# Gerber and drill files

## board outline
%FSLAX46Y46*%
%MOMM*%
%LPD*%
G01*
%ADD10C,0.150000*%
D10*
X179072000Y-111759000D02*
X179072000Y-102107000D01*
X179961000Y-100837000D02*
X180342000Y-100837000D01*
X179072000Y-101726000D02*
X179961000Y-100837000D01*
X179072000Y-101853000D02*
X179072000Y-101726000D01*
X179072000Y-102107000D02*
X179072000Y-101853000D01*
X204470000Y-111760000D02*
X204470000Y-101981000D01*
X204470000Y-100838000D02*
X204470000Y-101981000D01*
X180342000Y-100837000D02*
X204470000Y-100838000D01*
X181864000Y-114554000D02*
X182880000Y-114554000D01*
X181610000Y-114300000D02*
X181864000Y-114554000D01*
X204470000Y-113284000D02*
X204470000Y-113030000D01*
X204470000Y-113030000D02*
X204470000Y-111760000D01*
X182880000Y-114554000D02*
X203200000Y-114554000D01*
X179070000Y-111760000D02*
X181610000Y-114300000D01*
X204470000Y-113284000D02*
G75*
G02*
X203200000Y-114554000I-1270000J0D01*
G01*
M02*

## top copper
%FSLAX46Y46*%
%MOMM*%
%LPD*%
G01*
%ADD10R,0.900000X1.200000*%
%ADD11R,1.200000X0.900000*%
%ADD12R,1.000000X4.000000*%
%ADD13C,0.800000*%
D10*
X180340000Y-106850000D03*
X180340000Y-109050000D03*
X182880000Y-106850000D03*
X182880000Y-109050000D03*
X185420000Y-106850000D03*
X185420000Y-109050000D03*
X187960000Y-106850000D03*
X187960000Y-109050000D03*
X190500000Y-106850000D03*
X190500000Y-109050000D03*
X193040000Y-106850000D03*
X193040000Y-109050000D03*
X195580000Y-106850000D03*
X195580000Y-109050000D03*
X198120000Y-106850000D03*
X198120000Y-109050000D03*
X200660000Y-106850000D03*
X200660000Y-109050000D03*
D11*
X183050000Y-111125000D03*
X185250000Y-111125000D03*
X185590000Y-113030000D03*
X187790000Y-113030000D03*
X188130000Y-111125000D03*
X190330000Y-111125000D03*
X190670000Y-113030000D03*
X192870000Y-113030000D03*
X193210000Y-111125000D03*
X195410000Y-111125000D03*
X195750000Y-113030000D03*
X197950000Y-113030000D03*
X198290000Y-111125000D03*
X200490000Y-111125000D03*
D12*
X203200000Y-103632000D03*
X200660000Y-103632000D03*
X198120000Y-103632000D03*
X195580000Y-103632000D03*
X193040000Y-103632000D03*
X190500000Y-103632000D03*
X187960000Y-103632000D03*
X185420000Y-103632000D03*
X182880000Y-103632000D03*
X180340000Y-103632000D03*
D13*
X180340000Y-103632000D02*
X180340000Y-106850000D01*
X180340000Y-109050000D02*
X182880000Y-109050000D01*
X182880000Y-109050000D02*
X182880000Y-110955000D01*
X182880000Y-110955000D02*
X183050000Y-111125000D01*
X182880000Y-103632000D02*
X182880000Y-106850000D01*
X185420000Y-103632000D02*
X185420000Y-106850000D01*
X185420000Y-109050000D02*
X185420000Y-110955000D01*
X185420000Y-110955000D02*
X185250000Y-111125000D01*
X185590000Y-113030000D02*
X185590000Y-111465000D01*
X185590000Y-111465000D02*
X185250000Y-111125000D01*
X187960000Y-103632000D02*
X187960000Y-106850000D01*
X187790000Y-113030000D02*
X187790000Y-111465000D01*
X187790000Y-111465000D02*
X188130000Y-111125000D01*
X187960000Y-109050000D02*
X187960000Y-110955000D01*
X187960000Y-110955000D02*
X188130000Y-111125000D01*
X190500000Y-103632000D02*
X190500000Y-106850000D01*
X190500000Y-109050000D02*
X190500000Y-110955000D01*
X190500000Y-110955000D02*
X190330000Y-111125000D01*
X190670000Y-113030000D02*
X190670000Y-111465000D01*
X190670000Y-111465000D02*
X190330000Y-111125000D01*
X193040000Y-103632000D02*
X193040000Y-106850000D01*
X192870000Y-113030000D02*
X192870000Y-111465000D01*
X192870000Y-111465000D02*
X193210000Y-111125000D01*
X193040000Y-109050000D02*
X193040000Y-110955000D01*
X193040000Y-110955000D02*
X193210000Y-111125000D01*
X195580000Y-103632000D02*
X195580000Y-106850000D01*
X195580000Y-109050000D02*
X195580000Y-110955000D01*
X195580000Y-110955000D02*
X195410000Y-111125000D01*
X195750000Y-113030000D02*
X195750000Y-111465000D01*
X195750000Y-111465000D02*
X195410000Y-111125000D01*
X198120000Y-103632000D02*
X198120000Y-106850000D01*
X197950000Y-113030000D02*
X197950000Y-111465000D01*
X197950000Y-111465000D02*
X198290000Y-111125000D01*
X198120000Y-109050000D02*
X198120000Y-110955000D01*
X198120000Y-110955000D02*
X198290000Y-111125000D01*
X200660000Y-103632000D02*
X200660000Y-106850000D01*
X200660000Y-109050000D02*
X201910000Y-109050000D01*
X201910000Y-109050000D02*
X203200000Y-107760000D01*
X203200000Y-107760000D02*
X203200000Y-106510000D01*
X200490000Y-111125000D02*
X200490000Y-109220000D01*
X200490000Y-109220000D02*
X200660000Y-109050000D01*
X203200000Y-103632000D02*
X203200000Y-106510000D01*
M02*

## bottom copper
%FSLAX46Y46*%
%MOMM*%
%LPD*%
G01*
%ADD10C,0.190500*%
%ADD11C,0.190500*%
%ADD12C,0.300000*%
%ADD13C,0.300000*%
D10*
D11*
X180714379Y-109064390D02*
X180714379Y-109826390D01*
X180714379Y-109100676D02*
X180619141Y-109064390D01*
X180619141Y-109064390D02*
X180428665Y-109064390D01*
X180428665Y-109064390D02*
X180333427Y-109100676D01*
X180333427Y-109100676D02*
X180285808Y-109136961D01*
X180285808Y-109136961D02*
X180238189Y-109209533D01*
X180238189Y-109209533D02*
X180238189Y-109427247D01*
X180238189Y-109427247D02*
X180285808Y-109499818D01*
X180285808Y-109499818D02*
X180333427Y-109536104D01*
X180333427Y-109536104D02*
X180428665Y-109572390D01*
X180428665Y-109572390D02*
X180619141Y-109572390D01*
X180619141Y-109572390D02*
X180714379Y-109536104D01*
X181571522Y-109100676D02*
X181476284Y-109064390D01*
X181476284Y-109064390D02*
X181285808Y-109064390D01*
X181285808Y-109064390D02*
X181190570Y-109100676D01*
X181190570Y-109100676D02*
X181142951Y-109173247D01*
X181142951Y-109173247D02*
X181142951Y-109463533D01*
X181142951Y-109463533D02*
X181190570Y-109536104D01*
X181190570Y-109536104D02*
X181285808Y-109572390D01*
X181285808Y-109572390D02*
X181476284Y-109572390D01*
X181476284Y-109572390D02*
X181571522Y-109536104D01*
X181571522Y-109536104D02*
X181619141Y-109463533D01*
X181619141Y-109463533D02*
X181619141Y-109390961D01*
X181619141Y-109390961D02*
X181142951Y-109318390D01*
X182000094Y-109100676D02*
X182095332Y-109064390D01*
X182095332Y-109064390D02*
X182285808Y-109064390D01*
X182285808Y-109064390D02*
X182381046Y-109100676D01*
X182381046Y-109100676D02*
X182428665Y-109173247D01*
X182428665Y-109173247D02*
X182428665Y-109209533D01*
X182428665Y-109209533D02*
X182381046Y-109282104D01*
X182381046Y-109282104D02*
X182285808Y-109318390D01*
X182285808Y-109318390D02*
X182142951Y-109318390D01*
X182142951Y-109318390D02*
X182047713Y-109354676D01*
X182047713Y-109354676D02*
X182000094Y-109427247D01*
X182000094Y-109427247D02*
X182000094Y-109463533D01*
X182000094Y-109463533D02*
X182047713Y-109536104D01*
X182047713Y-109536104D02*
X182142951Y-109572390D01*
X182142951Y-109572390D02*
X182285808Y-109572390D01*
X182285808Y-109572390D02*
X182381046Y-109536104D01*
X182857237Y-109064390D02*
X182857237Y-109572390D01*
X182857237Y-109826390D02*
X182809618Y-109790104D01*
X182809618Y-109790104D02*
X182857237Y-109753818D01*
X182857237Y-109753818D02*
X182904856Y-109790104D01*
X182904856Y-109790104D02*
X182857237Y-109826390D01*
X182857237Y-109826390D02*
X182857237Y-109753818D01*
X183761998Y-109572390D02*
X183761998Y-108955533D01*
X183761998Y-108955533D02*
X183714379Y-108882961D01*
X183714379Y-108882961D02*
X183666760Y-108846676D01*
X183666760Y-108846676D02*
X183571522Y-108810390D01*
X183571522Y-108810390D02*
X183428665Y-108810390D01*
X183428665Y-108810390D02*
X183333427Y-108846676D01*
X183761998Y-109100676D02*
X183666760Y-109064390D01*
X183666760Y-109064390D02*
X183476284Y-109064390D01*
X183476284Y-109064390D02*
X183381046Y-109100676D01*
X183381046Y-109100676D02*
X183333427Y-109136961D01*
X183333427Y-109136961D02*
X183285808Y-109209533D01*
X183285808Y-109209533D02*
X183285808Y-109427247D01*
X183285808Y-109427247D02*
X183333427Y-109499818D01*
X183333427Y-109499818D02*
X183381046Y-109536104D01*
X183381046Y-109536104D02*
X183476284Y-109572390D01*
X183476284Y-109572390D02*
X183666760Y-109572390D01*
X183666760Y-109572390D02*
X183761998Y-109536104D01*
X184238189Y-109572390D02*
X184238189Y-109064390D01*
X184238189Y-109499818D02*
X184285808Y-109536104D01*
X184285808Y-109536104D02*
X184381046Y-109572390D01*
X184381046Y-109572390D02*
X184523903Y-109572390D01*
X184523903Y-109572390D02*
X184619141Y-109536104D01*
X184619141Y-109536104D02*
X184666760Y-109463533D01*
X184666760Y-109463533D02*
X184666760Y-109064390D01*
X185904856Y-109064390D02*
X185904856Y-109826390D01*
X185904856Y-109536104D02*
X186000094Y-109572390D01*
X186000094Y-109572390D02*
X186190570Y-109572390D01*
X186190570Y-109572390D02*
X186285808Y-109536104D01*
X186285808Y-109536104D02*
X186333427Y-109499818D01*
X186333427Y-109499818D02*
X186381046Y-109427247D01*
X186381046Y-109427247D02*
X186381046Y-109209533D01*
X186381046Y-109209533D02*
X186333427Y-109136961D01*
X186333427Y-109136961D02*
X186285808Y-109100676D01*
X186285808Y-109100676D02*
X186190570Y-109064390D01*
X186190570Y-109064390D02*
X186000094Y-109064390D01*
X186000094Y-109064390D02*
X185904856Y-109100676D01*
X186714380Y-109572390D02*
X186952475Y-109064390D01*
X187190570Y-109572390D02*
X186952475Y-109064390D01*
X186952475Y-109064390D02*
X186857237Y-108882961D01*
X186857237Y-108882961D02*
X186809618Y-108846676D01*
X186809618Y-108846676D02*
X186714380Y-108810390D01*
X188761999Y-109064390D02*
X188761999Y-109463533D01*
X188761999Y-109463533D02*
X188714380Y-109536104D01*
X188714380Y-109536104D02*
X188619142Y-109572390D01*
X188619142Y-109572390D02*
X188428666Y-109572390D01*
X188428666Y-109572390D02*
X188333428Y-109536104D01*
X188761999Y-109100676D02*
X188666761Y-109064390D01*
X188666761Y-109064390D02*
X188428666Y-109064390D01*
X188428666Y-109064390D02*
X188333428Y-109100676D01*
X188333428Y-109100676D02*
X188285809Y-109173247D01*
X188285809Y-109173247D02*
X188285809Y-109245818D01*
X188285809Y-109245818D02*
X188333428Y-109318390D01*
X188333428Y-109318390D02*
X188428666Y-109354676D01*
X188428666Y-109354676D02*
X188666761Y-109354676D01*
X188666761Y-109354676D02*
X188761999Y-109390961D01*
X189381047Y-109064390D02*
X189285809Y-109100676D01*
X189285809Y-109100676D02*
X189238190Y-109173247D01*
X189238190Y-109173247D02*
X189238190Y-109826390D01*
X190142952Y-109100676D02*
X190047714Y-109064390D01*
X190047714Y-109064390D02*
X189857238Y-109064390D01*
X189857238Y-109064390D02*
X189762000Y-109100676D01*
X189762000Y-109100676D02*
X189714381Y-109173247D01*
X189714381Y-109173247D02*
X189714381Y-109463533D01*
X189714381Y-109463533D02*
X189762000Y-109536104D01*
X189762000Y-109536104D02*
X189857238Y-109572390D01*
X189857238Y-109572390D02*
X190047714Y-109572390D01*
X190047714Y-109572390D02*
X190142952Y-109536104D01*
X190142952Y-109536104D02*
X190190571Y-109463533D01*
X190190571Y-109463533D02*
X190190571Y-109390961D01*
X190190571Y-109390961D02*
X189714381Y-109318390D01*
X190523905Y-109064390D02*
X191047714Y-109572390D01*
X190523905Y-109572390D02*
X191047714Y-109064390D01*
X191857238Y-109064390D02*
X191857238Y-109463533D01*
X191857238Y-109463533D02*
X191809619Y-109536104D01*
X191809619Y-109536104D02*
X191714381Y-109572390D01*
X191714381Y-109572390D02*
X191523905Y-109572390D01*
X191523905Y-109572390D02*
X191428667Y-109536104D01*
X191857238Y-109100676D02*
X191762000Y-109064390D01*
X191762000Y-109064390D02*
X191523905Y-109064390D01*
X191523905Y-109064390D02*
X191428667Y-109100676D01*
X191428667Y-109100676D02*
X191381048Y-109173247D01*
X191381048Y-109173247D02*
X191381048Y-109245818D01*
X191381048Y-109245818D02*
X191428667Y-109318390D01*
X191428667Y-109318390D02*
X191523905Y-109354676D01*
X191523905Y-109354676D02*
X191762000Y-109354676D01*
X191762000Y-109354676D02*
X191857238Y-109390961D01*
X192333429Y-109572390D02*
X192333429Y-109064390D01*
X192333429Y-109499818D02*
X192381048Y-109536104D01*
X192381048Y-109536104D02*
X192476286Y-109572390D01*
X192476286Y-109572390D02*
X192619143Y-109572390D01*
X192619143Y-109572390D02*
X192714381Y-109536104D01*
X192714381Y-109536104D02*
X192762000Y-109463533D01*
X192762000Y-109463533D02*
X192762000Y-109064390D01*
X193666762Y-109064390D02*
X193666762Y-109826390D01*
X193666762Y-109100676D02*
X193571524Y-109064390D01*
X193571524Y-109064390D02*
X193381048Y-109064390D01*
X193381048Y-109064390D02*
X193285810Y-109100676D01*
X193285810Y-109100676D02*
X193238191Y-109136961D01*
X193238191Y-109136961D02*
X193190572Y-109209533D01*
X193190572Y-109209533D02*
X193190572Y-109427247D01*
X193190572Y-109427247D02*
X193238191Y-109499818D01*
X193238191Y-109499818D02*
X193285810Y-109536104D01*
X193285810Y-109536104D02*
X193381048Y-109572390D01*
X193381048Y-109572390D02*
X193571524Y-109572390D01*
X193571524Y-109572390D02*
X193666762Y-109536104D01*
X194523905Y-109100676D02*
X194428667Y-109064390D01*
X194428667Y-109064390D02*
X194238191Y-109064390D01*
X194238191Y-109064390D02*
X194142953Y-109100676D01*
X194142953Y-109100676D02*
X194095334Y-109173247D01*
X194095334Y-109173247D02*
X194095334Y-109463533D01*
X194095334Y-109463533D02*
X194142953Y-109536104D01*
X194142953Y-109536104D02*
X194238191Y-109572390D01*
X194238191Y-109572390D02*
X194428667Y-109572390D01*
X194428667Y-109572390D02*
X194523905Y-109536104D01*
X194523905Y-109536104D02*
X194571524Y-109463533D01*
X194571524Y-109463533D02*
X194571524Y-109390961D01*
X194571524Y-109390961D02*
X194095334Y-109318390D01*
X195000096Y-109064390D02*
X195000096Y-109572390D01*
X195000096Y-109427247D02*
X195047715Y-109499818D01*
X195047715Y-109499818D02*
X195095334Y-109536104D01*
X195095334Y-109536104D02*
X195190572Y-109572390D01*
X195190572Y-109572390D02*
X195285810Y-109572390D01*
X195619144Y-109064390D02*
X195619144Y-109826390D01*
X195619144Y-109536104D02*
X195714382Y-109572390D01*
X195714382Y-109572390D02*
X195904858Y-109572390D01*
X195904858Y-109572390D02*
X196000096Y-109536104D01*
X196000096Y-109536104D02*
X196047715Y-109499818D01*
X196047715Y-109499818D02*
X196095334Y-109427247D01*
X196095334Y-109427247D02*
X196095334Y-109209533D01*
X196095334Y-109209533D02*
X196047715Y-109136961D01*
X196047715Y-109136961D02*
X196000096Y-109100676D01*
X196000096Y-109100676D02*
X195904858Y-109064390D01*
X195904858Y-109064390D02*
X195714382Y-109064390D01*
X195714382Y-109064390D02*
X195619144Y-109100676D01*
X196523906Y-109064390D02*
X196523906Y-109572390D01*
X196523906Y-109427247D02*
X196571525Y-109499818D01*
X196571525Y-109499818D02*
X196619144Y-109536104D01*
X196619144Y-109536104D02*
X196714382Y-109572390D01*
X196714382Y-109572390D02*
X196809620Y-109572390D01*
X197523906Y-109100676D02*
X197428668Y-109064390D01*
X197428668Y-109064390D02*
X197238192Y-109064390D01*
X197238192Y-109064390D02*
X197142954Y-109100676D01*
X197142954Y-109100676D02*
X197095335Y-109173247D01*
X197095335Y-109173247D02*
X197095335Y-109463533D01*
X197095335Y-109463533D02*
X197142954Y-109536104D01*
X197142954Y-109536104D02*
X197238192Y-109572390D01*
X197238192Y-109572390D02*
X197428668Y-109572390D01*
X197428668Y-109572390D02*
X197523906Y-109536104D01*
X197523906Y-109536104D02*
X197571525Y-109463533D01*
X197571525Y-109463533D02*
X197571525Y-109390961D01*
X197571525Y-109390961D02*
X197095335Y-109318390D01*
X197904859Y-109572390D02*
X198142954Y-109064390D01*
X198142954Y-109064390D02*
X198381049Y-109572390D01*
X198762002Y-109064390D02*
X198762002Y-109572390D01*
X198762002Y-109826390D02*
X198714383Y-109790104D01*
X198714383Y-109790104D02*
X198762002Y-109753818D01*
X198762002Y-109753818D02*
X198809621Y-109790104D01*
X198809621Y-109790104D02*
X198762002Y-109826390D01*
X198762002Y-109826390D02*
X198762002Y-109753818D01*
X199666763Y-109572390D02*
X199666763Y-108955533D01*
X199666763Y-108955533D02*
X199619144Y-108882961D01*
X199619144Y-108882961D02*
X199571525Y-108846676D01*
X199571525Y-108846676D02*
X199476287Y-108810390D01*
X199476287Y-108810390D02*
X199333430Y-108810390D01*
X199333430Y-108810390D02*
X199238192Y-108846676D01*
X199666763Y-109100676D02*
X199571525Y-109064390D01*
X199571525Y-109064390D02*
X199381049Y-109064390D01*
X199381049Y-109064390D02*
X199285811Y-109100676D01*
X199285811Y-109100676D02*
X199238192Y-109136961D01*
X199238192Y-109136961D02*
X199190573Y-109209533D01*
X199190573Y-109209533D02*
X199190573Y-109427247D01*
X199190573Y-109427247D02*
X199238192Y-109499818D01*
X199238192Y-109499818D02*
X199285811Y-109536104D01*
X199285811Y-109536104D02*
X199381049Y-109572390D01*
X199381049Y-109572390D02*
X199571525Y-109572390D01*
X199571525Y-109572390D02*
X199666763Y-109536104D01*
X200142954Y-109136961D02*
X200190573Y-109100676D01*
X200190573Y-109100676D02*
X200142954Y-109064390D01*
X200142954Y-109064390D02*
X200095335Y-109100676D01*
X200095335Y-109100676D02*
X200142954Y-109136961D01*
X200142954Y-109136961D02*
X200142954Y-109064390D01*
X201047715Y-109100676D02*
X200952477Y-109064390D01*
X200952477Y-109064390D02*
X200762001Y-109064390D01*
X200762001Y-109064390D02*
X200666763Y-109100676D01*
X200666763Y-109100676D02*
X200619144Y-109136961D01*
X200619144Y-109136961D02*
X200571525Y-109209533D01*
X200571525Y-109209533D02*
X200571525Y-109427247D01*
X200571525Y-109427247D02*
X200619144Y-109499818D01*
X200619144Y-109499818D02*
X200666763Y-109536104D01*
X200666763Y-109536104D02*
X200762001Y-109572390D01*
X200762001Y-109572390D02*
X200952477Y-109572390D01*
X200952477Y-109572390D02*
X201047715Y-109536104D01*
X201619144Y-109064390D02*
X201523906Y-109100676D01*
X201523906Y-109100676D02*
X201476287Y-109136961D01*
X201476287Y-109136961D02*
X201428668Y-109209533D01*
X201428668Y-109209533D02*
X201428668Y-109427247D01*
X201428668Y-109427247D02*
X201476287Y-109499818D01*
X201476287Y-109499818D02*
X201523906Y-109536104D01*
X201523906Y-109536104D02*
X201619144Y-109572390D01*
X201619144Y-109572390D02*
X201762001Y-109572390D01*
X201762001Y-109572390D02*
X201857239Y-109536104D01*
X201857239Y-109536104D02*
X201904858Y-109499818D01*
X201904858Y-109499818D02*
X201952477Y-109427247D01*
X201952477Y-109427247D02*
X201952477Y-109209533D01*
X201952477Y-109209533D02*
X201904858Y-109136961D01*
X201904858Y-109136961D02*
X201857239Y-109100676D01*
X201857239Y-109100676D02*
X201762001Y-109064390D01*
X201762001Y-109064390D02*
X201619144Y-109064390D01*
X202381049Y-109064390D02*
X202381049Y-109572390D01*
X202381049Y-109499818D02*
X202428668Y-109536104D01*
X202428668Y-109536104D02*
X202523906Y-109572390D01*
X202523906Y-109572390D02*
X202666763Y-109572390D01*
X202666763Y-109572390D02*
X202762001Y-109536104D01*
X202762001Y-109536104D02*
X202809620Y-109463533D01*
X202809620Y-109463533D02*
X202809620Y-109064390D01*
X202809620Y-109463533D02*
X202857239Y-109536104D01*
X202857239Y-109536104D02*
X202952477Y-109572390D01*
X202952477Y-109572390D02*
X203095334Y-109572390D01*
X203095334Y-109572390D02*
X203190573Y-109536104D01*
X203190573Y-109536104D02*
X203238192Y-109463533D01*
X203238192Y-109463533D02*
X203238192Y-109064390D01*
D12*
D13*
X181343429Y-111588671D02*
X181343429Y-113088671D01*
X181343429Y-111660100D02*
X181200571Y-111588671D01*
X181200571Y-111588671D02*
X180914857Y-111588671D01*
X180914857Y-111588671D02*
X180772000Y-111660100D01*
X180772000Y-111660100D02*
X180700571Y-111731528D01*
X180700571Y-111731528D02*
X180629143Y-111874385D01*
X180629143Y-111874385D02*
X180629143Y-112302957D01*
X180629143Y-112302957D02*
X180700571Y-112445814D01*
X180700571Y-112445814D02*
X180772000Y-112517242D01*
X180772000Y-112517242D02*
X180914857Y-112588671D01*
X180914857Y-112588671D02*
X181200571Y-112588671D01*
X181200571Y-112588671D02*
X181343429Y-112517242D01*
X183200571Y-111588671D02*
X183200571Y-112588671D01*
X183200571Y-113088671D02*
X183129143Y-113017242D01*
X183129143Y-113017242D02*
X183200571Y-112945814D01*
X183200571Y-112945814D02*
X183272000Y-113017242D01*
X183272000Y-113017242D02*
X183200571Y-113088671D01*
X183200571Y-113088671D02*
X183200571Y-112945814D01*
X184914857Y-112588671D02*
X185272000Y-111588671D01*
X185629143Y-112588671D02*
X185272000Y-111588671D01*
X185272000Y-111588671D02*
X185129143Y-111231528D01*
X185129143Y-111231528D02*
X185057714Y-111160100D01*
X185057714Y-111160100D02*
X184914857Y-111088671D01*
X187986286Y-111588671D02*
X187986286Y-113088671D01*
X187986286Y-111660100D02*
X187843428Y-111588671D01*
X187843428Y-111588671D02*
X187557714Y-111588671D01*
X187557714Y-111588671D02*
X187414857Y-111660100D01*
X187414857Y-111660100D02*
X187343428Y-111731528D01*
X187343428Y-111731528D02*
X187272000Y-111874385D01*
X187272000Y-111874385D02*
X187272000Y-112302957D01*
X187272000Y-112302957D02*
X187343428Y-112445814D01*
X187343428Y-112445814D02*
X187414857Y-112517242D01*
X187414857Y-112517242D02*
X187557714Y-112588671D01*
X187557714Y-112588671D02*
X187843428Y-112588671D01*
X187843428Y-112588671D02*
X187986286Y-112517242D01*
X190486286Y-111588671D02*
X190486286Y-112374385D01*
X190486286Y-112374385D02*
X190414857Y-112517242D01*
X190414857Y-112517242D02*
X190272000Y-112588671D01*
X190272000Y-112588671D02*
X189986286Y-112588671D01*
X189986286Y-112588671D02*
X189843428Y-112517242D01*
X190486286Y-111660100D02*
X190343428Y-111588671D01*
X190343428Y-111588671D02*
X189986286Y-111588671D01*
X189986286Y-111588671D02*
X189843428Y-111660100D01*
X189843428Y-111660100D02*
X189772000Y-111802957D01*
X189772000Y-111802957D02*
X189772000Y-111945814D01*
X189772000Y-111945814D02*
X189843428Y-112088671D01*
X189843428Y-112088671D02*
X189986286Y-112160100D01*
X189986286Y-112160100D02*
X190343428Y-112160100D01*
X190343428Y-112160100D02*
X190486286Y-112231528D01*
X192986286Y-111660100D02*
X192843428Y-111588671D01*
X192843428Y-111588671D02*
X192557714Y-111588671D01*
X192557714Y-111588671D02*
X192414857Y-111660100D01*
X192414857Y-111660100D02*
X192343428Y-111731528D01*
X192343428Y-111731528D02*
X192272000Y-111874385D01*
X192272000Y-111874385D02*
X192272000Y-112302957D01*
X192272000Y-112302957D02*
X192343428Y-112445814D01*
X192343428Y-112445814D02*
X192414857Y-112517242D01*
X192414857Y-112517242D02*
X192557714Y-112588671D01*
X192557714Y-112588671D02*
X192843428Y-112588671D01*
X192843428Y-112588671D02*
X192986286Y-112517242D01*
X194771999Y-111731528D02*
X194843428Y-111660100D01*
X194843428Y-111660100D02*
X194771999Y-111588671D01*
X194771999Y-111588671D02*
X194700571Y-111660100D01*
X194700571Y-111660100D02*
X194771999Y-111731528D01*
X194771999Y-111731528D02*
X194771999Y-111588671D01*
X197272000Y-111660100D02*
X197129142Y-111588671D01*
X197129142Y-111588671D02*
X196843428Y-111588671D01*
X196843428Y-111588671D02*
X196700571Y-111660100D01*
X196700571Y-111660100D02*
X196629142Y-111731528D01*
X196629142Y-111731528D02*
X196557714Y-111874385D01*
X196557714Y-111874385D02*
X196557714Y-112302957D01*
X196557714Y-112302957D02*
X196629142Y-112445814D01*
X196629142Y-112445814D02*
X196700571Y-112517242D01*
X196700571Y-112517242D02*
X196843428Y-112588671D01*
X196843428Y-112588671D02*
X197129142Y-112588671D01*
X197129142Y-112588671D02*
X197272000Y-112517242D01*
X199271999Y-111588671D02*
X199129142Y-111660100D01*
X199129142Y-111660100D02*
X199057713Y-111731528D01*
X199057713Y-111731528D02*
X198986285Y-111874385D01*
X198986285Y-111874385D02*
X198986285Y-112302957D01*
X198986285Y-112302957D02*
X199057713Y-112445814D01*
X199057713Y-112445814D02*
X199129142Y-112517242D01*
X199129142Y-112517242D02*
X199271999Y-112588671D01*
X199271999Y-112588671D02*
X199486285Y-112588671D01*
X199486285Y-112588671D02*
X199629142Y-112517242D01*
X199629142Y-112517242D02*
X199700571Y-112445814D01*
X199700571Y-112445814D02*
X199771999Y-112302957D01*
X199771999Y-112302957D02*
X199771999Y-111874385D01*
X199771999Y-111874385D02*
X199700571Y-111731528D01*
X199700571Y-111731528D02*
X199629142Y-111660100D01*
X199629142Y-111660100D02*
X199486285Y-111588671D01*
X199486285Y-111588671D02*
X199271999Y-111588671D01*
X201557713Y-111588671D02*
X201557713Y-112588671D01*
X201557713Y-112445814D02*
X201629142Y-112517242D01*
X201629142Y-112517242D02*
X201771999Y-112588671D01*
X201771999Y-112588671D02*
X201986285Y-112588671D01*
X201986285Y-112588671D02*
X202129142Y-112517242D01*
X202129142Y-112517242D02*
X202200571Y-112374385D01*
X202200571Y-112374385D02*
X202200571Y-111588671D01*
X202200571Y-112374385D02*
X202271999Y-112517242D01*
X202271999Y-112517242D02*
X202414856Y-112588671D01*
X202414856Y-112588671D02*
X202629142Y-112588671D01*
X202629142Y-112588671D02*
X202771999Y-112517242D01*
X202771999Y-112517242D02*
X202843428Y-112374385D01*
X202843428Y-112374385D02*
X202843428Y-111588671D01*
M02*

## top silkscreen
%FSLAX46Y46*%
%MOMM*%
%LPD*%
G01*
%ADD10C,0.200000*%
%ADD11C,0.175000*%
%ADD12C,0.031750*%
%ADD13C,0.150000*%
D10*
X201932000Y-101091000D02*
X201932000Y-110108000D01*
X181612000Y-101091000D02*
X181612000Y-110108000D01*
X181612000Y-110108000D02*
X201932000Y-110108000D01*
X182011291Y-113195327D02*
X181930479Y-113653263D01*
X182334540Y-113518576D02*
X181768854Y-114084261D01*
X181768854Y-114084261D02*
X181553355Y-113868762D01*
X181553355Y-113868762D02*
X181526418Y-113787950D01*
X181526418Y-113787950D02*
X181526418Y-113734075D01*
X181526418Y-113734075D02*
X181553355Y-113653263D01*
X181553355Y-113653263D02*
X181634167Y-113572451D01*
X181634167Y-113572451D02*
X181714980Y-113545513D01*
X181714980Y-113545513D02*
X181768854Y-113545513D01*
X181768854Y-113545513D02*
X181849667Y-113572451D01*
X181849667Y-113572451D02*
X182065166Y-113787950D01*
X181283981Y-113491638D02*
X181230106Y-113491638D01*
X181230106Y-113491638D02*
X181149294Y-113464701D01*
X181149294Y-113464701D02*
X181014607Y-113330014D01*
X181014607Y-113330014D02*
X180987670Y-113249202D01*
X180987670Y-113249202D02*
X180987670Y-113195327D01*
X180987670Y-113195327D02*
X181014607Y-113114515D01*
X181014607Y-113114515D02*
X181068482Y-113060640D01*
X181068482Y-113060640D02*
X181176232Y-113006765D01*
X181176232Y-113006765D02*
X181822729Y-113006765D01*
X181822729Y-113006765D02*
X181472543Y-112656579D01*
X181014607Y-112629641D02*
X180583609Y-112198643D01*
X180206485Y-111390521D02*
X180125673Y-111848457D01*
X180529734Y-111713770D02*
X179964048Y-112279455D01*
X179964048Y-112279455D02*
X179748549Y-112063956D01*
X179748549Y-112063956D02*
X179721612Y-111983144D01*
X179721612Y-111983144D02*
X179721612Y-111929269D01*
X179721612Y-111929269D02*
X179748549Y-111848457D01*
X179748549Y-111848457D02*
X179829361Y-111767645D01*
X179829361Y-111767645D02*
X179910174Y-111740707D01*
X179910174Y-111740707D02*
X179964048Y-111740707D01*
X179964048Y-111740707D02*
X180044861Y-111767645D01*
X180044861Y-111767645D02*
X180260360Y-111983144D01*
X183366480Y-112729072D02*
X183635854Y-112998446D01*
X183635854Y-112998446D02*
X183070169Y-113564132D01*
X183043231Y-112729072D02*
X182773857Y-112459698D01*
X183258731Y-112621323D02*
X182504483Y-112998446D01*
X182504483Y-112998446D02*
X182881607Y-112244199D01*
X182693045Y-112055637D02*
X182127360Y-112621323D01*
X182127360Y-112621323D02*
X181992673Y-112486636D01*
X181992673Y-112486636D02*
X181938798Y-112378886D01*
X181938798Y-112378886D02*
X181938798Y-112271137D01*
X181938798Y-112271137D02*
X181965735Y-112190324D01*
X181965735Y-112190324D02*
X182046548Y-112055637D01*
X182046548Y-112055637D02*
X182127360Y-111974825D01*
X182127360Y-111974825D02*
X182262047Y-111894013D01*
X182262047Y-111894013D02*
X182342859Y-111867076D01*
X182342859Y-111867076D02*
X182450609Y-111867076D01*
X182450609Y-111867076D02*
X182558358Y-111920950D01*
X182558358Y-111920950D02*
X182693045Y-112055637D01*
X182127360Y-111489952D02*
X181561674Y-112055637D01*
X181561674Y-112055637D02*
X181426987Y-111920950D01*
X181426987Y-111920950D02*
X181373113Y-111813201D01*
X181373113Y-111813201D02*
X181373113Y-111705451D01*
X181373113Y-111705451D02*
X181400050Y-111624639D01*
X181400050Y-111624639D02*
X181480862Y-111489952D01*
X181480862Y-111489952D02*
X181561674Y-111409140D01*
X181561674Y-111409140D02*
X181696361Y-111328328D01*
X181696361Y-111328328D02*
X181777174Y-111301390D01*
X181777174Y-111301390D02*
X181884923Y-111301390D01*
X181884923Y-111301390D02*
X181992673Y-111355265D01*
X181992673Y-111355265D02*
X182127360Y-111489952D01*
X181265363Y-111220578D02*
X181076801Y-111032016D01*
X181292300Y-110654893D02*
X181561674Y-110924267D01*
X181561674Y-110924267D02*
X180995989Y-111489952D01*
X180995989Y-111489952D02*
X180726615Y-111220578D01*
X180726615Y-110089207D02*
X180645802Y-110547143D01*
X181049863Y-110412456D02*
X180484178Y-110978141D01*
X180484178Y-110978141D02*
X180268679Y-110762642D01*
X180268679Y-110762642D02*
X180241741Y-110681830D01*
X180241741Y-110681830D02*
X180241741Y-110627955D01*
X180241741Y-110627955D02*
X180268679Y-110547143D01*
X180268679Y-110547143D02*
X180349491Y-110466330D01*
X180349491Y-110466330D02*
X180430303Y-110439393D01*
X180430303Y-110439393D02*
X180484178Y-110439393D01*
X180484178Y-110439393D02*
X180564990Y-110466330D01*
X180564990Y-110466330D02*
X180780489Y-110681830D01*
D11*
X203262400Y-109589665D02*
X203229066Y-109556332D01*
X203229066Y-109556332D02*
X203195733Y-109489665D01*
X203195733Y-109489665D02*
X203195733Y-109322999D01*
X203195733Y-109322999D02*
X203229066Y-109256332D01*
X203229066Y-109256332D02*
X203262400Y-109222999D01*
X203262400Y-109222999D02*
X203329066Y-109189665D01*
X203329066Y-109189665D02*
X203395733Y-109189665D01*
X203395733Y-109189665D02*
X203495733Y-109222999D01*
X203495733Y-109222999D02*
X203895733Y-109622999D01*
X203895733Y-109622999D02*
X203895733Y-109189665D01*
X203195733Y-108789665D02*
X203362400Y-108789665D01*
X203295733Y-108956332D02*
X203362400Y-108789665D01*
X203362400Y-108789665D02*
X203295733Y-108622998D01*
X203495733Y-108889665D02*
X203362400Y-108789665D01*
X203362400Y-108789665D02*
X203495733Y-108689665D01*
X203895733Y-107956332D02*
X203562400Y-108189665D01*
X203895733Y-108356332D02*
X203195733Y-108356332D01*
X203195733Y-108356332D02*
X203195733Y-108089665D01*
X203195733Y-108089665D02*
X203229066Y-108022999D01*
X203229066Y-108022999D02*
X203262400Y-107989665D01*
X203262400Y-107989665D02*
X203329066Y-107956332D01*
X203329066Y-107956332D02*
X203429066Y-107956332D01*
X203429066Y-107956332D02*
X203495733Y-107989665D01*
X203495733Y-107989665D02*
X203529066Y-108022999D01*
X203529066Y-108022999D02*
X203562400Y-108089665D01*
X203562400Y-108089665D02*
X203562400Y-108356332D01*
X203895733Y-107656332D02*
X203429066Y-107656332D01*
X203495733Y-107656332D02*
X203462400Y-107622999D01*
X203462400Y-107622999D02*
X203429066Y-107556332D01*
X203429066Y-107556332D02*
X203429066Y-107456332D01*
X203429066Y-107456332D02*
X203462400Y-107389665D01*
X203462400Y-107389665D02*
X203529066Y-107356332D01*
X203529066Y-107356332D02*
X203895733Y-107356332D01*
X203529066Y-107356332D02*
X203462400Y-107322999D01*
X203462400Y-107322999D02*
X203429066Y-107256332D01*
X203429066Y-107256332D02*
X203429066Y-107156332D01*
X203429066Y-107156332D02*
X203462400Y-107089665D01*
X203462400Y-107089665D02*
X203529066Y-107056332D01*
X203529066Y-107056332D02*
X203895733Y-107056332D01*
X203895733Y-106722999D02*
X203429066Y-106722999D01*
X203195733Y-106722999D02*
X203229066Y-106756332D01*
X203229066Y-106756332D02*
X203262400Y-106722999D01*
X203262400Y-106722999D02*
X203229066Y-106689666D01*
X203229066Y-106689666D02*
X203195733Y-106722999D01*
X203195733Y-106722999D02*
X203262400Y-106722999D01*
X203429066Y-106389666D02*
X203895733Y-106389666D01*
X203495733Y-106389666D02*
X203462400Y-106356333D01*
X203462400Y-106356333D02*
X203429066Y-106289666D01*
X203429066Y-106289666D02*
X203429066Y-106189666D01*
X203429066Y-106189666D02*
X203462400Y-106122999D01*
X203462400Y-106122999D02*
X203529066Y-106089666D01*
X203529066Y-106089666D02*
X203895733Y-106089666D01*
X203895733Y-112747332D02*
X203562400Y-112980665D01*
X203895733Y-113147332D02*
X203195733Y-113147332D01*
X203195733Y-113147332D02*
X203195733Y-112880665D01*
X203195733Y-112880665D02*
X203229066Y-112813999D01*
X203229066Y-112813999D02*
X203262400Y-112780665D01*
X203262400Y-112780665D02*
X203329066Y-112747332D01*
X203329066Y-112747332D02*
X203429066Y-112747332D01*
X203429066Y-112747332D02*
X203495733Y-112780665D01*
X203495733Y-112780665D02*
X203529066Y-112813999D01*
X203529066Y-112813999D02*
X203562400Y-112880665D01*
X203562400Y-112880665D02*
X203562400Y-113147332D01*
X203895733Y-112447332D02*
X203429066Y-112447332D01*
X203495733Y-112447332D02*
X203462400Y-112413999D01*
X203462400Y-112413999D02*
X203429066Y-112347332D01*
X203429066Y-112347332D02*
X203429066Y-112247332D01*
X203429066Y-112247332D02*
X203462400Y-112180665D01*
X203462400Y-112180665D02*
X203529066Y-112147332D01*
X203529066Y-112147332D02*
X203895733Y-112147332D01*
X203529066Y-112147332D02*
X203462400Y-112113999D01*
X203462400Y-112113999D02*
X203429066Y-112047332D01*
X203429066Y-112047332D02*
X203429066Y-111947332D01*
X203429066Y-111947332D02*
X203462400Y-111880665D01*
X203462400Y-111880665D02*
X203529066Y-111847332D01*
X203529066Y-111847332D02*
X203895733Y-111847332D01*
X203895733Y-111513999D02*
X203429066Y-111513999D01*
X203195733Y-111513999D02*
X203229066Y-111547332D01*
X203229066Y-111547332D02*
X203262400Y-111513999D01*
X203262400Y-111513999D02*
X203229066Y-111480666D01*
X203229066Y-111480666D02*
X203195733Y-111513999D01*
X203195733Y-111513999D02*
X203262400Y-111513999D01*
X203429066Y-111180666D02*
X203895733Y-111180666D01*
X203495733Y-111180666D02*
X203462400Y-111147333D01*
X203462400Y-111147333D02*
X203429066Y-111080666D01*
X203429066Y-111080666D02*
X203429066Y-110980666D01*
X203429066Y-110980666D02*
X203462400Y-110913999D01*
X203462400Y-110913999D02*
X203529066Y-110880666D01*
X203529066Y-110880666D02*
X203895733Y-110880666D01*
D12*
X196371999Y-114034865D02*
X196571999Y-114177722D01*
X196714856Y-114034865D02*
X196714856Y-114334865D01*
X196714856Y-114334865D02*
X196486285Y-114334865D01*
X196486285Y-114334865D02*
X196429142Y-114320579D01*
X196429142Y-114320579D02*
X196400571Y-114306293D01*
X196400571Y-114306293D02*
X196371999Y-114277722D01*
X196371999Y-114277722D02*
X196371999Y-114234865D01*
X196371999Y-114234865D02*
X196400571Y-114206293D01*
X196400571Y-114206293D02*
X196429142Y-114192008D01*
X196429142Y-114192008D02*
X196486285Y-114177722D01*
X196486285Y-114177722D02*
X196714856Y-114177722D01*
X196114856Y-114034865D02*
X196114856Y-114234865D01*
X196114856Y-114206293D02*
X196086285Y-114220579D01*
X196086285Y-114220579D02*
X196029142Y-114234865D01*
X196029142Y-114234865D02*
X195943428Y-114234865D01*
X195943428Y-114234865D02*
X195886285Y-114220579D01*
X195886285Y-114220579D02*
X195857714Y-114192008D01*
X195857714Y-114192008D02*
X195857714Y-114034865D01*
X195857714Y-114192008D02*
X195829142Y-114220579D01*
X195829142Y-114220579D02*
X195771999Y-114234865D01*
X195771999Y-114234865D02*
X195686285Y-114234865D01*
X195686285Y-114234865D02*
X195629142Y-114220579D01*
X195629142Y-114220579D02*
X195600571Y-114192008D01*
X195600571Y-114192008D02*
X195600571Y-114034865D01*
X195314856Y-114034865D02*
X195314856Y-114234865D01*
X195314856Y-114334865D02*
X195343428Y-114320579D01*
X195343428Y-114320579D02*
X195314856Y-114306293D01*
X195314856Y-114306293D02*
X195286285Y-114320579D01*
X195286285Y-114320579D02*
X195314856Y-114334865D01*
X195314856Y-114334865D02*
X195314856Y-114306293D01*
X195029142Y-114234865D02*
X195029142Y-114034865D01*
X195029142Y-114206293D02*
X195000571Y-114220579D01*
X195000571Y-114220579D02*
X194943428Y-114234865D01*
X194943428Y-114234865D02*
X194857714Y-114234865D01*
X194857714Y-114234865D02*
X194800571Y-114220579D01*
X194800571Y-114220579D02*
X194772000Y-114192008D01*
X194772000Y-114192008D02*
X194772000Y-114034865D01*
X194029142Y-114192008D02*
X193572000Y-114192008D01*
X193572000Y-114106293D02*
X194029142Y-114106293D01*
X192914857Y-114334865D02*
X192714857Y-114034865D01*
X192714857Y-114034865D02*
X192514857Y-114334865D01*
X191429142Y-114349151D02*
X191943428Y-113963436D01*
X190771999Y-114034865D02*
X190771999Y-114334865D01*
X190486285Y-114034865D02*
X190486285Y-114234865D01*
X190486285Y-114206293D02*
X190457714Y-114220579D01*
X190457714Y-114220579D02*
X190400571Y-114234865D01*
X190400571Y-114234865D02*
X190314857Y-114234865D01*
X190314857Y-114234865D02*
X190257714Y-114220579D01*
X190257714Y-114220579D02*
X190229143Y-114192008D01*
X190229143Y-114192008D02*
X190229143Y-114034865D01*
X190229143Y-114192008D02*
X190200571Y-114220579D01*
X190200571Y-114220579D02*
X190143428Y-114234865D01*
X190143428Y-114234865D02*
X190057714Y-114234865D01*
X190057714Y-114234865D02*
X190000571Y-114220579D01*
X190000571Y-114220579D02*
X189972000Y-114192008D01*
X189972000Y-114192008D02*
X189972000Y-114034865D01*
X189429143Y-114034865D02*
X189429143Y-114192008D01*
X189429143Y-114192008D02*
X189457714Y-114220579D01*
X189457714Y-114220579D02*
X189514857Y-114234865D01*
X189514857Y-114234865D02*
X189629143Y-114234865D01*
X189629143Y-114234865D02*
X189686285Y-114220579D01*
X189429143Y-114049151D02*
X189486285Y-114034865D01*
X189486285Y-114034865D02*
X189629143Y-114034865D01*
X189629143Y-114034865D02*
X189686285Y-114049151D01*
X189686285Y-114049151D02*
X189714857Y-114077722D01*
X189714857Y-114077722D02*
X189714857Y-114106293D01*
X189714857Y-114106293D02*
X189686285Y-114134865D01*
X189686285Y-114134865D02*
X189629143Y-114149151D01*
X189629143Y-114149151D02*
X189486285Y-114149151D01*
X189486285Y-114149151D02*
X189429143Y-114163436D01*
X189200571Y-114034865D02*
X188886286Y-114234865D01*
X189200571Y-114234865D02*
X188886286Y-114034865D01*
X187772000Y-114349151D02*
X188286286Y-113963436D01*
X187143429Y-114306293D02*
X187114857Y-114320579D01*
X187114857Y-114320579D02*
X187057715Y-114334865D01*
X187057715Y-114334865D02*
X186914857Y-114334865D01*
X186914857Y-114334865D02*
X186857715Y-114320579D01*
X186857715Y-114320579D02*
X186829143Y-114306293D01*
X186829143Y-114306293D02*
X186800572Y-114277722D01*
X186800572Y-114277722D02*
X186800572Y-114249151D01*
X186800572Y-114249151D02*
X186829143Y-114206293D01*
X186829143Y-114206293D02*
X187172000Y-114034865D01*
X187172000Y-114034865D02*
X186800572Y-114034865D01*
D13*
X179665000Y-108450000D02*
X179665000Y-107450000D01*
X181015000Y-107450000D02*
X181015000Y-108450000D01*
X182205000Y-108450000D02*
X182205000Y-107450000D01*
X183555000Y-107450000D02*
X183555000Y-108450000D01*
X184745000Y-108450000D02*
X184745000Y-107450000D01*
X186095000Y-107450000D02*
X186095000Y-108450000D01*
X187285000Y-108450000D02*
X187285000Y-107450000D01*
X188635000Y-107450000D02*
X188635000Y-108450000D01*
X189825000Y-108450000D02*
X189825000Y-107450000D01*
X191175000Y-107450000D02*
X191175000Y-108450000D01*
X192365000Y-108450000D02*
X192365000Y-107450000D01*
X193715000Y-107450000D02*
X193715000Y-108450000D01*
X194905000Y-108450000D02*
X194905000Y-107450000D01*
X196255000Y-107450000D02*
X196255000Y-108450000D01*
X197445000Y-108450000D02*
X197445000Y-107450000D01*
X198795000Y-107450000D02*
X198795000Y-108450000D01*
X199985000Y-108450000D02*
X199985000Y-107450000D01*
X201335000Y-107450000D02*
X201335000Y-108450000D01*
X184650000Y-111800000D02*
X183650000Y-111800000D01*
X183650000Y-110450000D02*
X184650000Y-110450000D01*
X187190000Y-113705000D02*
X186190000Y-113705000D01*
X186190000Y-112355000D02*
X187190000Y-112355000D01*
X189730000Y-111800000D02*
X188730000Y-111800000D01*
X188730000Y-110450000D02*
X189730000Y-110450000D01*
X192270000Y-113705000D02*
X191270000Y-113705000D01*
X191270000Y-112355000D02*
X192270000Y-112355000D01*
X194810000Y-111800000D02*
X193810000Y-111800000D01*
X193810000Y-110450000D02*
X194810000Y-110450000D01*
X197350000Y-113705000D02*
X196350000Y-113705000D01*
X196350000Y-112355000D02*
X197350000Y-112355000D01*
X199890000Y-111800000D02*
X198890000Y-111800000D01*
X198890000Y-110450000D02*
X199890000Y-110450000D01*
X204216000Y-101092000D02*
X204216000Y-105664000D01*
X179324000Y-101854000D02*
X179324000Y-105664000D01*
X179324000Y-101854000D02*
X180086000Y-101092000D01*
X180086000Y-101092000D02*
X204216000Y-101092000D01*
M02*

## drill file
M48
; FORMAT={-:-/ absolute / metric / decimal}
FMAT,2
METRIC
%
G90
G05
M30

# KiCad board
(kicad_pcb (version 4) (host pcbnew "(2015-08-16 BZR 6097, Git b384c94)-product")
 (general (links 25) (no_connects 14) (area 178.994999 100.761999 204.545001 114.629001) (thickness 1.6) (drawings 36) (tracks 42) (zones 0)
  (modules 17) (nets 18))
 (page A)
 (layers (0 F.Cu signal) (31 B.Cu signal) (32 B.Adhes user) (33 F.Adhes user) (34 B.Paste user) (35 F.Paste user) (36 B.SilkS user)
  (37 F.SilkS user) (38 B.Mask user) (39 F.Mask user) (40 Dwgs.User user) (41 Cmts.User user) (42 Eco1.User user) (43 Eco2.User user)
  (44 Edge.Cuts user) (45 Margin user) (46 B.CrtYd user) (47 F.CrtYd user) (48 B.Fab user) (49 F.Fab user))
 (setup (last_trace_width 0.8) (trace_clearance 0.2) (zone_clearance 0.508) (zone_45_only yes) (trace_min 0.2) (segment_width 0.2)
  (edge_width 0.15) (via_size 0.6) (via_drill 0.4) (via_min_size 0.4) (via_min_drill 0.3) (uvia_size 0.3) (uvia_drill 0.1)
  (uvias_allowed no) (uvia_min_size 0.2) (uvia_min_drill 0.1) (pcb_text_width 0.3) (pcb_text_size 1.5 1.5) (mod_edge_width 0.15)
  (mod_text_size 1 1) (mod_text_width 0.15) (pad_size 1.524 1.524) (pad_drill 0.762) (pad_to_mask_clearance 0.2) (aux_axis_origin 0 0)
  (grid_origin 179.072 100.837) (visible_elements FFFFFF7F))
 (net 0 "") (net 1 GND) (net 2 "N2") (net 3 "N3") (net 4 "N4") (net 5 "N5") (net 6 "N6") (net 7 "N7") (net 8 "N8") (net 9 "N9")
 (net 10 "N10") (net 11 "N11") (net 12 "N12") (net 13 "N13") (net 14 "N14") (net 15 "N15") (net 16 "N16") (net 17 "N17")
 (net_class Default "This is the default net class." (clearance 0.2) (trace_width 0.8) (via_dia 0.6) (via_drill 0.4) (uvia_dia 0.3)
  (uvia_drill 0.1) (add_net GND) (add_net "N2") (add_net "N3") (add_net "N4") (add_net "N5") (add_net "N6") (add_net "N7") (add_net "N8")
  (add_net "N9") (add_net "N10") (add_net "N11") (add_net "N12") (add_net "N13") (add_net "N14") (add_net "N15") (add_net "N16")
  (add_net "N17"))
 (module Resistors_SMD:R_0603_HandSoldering (layer F.Cu) (at 180.34 107.95 270)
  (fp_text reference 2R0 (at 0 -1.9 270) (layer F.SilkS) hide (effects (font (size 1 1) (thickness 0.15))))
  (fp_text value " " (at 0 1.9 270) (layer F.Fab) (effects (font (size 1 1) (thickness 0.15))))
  (fp_line (start 0.5 0.675) (end -0.5 0.675) (layer F.SilkS) (width 0.15))
  (fp_line (start -0.5 -0.675) (end 0.5 -0.675) (layer F.SilkS) (width 0.15))
  (pad 1 smd rect (at -1.1 0 270) (size 1.2 0.9) (layers F.Cu F.Paste F.Mask) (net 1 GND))
  (pad 2 smd rect (at 1.1 0 270) (size 1.2 0.9) (layers F.Cu F.Paste F.Mask) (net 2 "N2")))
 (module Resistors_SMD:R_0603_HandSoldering (layer F.Cu) (at 182.88 107.95 270)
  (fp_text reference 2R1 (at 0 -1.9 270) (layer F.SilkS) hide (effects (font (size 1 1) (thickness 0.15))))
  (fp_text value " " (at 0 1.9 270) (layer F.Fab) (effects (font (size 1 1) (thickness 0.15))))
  (fp_line (start 0.5 0.675) (end -0.5 0.675) (layer F.SilkS) (width 0.15))
  (fp_line (start -0.5 -0.675) (end 0.5 -0.675) (layer F.SilkS) (width 0.15))
  (pad 1 smd rect (at -1.1 0 270) (size 1.2 0.9) (layers F.Cu F.Paste F.Mask) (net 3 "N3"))
  (pad 2 smd rect (at 1.1 0 270) (size 1.2 0.9) (layers F.Cu F.Paste F.Mask) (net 2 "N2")))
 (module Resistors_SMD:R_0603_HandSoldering (layer F.Cu) (at 185.42 107.95 270)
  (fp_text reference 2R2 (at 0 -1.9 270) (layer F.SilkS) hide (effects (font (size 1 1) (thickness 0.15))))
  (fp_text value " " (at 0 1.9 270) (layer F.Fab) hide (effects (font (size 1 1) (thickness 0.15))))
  (fp_line (start 0.5 0.675) (end -0.5 0.675) (layer F.SilkS) (width 0.15))
  (fp_line (start -0.5 -0.675) (end 0.5 -0.675) (layer F.SilkS) (width 0.15))
  (pad 1 smd rect (at -1.1 0 270) (size 1.2 0.9) (layers F.Cu F.Paste F.Mask) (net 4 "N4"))
  (pad 2 smd rect (at 1.1 0 270) (size 1.2 0.9) (layers F.Cu F.Paste F.Mask) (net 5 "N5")))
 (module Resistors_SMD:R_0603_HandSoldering (layer F.Cu) (at 187.96 107.95 270)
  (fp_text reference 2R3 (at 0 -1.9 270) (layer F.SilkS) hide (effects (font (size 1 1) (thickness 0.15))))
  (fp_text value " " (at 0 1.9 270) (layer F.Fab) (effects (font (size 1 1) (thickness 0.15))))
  (fp_line (start 0.5 0.675) (end -0.5 0.675) (layer F.SilkS) (width 0.15))
  (fp_line (start -0.5 -0.675) (end 0.5 -0.675) (layer F.SilkS) (width 0.15))
  (pad 1 smd rect (at -1.1 0 270) (size 1.2 0.9) (layers F.Cu F.Paste F.Mask) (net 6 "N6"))
  (pad 2 smd rect (at 1.1 0 270) (size 1.2 0.9) (layers F.Cu F.Paste F.Mask) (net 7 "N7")))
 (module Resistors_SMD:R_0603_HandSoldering (layer F.Cu) (at 190.5 107.95 270)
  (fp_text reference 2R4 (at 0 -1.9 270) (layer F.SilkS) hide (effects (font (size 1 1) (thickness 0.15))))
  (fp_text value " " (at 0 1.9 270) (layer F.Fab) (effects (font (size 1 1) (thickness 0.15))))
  (fp_line (start 0.5 0.675) (end -0.5 0.675) (layer F.SilkS) (width 0.15))
  (fp_line (start -0.5 -0.675) (end 0.5 -0.675) (layer F.SilkS) (width 0.15))
  (pad 1 smd rect (at -1.1 0 270) (size 1.2 0.9) (layers F.Cu F.Paste F.Mask) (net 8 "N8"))
  (pad 2 smd rect (at 1.1 0 270) (size 1.2 0.9) (layers F.Cu F.Paste F.Mask) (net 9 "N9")))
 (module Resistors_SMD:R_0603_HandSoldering (layer F.Cu) (at 193.04 107.95 270)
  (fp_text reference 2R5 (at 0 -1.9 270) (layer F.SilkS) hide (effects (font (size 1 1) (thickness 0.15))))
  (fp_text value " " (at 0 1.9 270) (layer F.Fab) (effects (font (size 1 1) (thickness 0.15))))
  (fp_line (start 0.5 0.675) (end -0.5 0.675) (layer F.SilkS) (width 0.15))
  (fp_line (start -0.5 -0.675) (end 0.5 -0.675) (layer F.SilkS) (width 0.15))
  (pad 1 smd rect (at -1.1 0 270) (size 1.2 0.9) (layers F.Cu F.Paste F.Mask) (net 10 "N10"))
  (pad 2 smd rect (at 1.1 0 270) (size 1.2 0.9) (layers F.Cu F.Paste F.Mask) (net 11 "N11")))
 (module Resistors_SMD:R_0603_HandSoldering (layer F.Cu) (at 195.58 107.95 270)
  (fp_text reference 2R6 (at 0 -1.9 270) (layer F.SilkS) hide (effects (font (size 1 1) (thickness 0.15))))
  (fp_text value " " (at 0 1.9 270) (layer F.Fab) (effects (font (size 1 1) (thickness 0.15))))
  (fp_line (start 0.5 0.675) (end -0.5 0.675) (layer F.SilkS) (width 0.15))
  (fp_line (start -0.5 -0.675) (end 0.5 -0.675) (layer F.SilkS) (width 0.15))
  (pad 1 smd rect (at -1.1 0 270) (size 1.2 0.9) (layers F.Cu F.Paste F.Mask) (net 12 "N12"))
  (pad 2 smd rect (at 1.1 0 270) (size 1.2 0.9) (layers F.Cu F.Paste F.Mask) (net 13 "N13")))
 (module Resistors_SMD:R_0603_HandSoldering (layer F.Cu) (at 198.12 107.95 270)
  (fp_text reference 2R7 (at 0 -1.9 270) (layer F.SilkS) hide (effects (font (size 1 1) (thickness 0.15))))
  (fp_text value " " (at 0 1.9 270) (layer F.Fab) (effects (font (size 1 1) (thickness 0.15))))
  (fp_line (start 0.5 0.675) (end -0.5 0.675) (layer F.SilkS) (width 0.15))
  (fp_line (start -0.5 -0.675) (end 0.5 -0.675) (layer F.SilkS) (width 0.15))
  (pad 1 smd rect (at -1.1 0 270) (size 1.2 0.9) (layers F.Cu F.Paste F.Mask) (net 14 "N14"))
  (pad 2 smd rect (at 1.1 0 270) (size 1.2 0.9) (layers F.Cu F.Paste F.Mask) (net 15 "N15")))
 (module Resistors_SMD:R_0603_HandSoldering (layer F.Cu) (at 200.66 107.95 270)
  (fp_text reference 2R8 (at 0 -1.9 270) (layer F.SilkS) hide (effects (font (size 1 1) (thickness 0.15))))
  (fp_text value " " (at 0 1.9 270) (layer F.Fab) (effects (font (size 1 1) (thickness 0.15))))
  (fp_line (start 0.5 0.675) (end -0.5 0.675) (layer F.SilkS) (width 0.15))
  (fp_line (start -0.5 -0.675) (end 0.5 -0.675) (layer F.SilkS) (width 0.15))
  (pad 1 smd rect (at -1.1 0 270) (size 1.2 0.9) (layers F.Cu F.Paste F.Mask) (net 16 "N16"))
  (pad 2 smd rect (at 1.1 0 270) (size 1.2 0.9) (layers F.Cu F.Paste F.Mask) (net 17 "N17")))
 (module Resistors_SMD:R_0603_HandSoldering (layer F.Cu) (at 184.15 111.125)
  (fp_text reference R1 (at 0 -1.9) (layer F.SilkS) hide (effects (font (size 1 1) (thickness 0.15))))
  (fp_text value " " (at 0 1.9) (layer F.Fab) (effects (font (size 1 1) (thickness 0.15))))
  (fp_line (start 0.5 0.675) (end -0.5 0.675) (layer F.SilkS) (width 0.15))
  (fp_line (start -0.5 -0.675) (end 0.5 -0.675) (layer F.SilkS) (width 0.15))
  (pad 1 smd rect (at -1.1 0) (size 1.2 0.9) (layers F.Cu F.Paste F.Mask) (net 2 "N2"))
  (pad 2 smd rect (at 1.1 0) (size 1.2 0.9) (layers F.Cu F.Paste F.Mask) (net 5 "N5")))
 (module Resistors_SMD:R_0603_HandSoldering (layer F.Cu) (at 186.69 113.03)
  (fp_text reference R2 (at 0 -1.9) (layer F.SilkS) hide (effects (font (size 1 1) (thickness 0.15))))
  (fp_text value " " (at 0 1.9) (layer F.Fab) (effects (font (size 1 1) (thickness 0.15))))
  (fp_line (start 0.5 0.675) (end -0.5 0.675) (layer F.SilkS) (width 0.15))
  (fp_line (start -0.5 -0.675) (end 0.5 -0.675) (layer F.SilkS) (width 0.15))
  (pad 1 smd rect (at -1.1 0) (size 1.2 0.9) (layers F.Cu F.Paste F.Mask) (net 5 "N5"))
  (pad 2 smd rect (at 1.1 0) (size 1.2 0.9) (layers F.Cu F.Paste F.Mask) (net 7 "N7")))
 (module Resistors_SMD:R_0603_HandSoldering (layer F.Cu) (at 189.23 111.125)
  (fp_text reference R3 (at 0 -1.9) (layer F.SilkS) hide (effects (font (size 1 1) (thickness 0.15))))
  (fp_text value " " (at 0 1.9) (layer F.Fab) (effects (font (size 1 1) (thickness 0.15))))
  (fp_line (start 0.5 0.675) (end -0.5 0.675) (layer F.SilkS) (width 0.15))
  (fp_line (start -0.5 -0.675) (end 0.5 -0.675) (layer F.SilkS) (width 0.15))
  (pad 1 smd rect (at -1.1 0) (size 1.2 0.9) (layers F.Cu F.Paste F.Mask) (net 7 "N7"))
  (pad 2 smd rect (at 1.1 0) (size 1.2 0.9) (layers F.Cu F.Paste F.Mask) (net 9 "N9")))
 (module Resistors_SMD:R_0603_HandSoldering (layer F.Cu) (at 191.77 113.03)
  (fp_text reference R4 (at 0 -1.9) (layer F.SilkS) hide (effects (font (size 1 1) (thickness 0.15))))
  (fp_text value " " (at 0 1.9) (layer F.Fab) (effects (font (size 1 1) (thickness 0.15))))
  (fp_line (start 0.5 0.675) (end -0.5 0.675) (layer F.SilkS) (width 0.15))
  (fp_line (start -0.5 -0.675) (end 0.5 -0.675) (layer F.SilkS) (width 0.15))
  (pad 1 smd rect (at -1.1 0) (size 1.2 0.9) (layers F.Cu F.Paste F.Mask) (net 9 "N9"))
  (pad 2 smd rect (at 1.1 0) (size 1.2 0.9) (layers F.Cu F.Paste F.Mask) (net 11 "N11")))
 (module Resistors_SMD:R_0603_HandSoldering (layer F.Cu) (at 194.31 111.125)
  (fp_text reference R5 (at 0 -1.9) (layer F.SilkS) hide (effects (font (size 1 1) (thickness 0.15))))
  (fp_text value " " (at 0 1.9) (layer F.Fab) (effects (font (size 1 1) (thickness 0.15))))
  (fp_line (start 0.5 0.675) (end -0.5 0.675) (layer F.SilkS) (width 0.15))
  (fp_line (start -0.5 -0.675) (end 0.5 -0.675) (layer F.SilkS) (width 0.15))
  (pad 1 smd rect (at -1.1 0) (size 1.2 0.9) (layers F.Cu F.Paste F.Mask) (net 11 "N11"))
  (pad 2 smd rect (at 1.1 0) (size 1.2 0.9) (layers F.Cu F.Paste F.Mask) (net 13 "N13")))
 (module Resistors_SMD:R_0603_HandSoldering (layer F.Cu) (at 196.85 113.03)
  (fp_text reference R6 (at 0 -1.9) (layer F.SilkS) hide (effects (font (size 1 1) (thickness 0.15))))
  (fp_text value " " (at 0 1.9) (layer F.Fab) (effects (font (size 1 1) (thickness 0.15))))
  (fp_line (start 0.5 0.675) (end -0.5 0.675) (layer F.SilkS) (width 0.15))
  (fp_line (start -0.5 -0.675) (end 0.5 -0.675) (layer F.SilkS) (width 0.15))
  (pad 1 smd rect (at -1.1 0) (size 1.2 0.9) (layers F.Cu F.Paste F.Mask) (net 13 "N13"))
  (pad 2 smd rect (at 1.1 0) (size 1.2 0.9) (layers F.Cu F.Paste F.Mask) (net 15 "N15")))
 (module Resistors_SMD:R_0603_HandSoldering (layer F.Cu) (at 199.39 111.125)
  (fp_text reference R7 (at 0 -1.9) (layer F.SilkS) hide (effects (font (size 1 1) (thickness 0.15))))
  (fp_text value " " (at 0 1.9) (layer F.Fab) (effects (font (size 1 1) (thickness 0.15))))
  (fp_line (start 0.5 0.675) (end -0.5 0.675) (layer F.SilkS) (width 0.15))
  (fp_line (start -0.5 -0.675) (end 0.5 -0.675) (layer F.SilkS) (width 0.15))
  (pad 1 smd rect (at -1.1 0) (size 1.2 0.9) (layers F.Cu F.Paste F.Mask) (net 15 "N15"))
  (pad 2 smd rect (at 1.1 0) (size 1.2 0.9) (layers F.Cu F.Paste F.Mask) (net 17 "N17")))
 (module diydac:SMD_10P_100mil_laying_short (layer F.Cu) (at 180.34 103.632)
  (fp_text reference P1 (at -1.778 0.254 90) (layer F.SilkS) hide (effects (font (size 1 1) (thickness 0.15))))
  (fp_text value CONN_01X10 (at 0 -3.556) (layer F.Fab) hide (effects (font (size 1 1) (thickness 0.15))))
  (fp_line (start 23.876 -2.54) (end 23.876 2.032) (layer F.SilkS) (width 0.15))
  (fp_line (start -1.016 -1.778) (end -1.016 2.032) (layer F.SilkS) (width 0.15))
  (fp_line (start -1.016 -1.778) (end -0.254 -2.54) (layer F.SilkS) (width 0.15))
  (fp_line (start -0.254 -2.54) (end 23.876 -2.54) (layer F.SilkS) (width 0.15))
  (pad 10 smd rect (at 22.86 0) (size 1 4) (layers F.Cu F.Paste F.Mask) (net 17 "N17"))
  (pad 9 smd rect (at 20.32 0) (size 1 4) (layers F.Cu F.Paste F.Mask) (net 16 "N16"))
  (pad 8 smd rect (at 17.78 0) (size 1 4) (layers F.Cu F.Paste F.Mask) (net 14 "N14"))
  (pad 7 smd rect (at 15.24 0) (size 1 4) (layers F.Cu F.Paste F.Mask) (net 12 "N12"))
  (pad 6 smd rect (at 12.7 0) (size 1 4) (layers F.Cu F.Paste F.Mask) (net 10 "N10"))
  (pad 5 smd rect (at 10.16 0) (size 1 4) (layers F.Cu F.Paste F.Mask) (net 8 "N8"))
  (pad 4 smd rect (at 7.62 0) (size 1 4) (layers F.Cu F.Paste F.Mask) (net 6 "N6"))
  (pad 3 smd rect (at 5.08 0) (size 1 4) (layers F.Cu F.Paste F.Mask) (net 4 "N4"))
  (pad 2 smd rect (at 2.54 0) (size 1 4) (layers F.Cu F.Paste F.Mask) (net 3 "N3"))
  (pad 1 smd rect (at 0 0) (size 1 4) (layers F.Cu F.Paste F.Mask) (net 1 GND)))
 (gr_line (start 201.932 101.091) (end 201.932 110.108) (layer F.SilkS) (width 0.2))
 (gr_line (start 181.612 101.091) (end 181.612 110.108) (layer F.SilkS) (width 0.2))
 (gr_line (start 179.072 111.759) (end 179.072 102.107) (layer Edge.Cuts) (width 0.15))
 (gr_line (start 179.961 100.837) (end 180.342 100.837) (layer Edge.Cuts) (width 0.15))
 (gr_line (start 179.072 101.726) (end 179.961 100.837) (layer Edge.Cuts) (width 0.15))
 (gr_line (start 179.072 101.853) (end 179.072 101.726) (layer Edge.Cuts) (width 0.15))
 (gr_line (start 179.072 102.107) (end 179.072 101.853) (layer Edge.Cuts) (width 0.15))
 (gr_line (start 204.47 111.76) (end 204.47 101.981) (angle 90) (layer Edge.Cuts) (width 0.15))
 (gr_line (start 204.47 100.838) (end 204.47 101.981) (angle 90) (layer Edge.Cuts) (width 0.15))
 (gr_line (start 180.342 100.837) (end 204.47 100.838) (angle 90) (layer Edge.Cuts) (width 0.15))
 (gr_line (start 181.864 114.554) (end 182.88 114.554) (angle 90) (layer Edge.Cuts) (width 0.15))
 (gr_line (start 181.61 114.3) (end 181.864 114.554) (angle 90) (layer Edge.Cuts) (width 0.15))
 (gr_line (start 204.47 113.284) (end 204.47 113.03) (angle 90) (layer Edge.Cuts) (width 0.15))
 (gr_line (start 181.612 110.108) (end 201.932 110.108) (angle 90) (layer F.SilkS) (width 0.2))
 (gr_line (start 204.47 113.03) (end 204.47 111.76) (angle 90) (layer Edge.Cuts) (width 0.15))
 (gr_line (start 182.88 114.554) (end 203.2 114.554) (angle 90) (layer Edge.Cuts) (width 0.15))
 (gr_line (start 179.07 111.76) (end 181.61 114.3) (angle 90) (layer Edge.Cuts) (width 0.15))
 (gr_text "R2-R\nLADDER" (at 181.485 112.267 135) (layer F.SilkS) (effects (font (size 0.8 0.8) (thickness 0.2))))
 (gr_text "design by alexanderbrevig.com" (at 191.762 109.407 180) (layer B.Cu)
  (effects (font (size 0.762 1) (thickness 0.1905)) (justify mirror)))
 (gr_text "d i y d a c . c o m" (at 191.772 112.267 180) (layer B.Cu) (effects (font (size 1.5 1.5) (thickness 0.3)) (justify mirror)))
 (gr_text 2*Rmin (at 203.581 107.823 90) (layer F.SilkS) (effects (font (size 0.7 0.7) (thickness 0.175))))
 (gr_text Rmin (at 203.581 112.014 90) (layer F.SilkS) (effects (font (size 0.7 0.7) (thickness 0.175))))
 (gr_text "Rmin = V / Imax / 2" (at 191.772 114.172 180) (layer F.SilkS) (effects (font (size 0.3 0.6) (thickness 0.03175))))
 (gr_arc (start 203.2 113.284) (end 204.47 113.284) (angle 90) (layer Edge.Cuts) (width 0.15))
 (segment (start 180.34 103.632) (end 180.34 106.85) (width 0.8) (layer F.Cu) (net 1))
 (segment (start 180.34 109.05) (end 182.88 109.05) (width 0.8) (layer F.Cu) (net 2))
 (segment (start 182.88 109.05) (end 182.88 110.955) (width 0.8) (layer F.Cu) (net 2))
 (segment (start 182.88 110.955) (end 183.05 111.125) (width 0.8) (layer F.Cu) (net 2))
 (segment (start 182.88 103.632) (end 182.88 106.85) (width 0.8) (layer F.Cu) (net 3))
 (segment (start 185.42 103.632) (end 185.42 106.85) (width 0.8) (layer F.Cu) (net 4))
 (segment (start 185.42 109.05) (end 185.42 110.955) (width 0.8) (layer F.Cu) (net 5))
 (segment (start 185.42 110.955) (end 185.25 111.125) (width 0.8) (layer F.Cu) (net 5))
 (segment (start 185.59 113.03) (end 185.59 111.465) (width 0.8) (layer F.Cu) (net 5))
 (segment (start 185.59 111.465) (end 185.25 111.125) (width 0.8) (layer F.Cu) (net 5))
 (segment (start 187.96 103.632) (end 187.96 106.85) (width 0.8) (layer F.Cu) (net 6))
 (segment (start 187.79 113.03) (end 187.79 111.465) (width 0.8) (layer F.Cu) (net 7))
 (segment (start 187.79 111.465) (end 188.13 111.125) (width 0.8) (layer F.Cu) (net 7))
 (segment (start 187.96 109.05) (end 187.96 110.955) (width 0.8) (layer F.Cu) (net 7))
 (segment (start 187.96 110.955) (end 188.13 111.125) (width 0.8) (layer F.Cu) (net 7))
 (segment (start 190.5 103.632) (end 190.5 106.85) (width 0.8) (layer F.Cu) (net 8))
 (segment (start 190.5 109.05) (end 190.5 110.955) (width 0.8) (layer F.Cu) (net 9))
 (segment (start 190.5 110.955) (end 190.33 111.125) (width 0.8) (layer F.Cu) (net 9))
 (segment (start 190.67 113.03) (end 190.67 111.465) (width 0.8) (layer F.Cu) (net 9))
 (segment (start 190.67 111.465) (end 190.33 111.125) (width 0.8) (layer F.Cu) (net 9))
 (segment (start 193.04 103.632) (end 193.04 106.85) (width 0.8) (layer F.Cu) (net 10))
 (segment (start 192.87 113.03) (end 192.87 111.465) (width 0.8) (layer F.Cu) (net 11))
 (segment (start 192.87 111.465) (end 193.21 111.125) (width 0.8) (layer F.Cu) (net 11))
 (segment (start 193.04 109.05) (end 193.04 110.955) (width 0.8) (layer F.Cu) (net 11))
 (segment (start 193.04 110.955) (end 193.21 111.125) (width 0.8) (layer F.Cu) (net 11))
 (segment (start 195.58 103.632) (end 195.58 106.85) (width 0.8) (layer F.Cu) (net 12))
 (segment (start 195.58 109.05) (end 195.58 110.955) (width 0.8) (layer F.Cu) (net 13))
 (segment (start 195.58 110.955) (end 195.41 111.125) (width 0.8) (layer F.Cu) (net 13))
 (segment (start 195.75 113.03) (end 195.75 111.465) (width 0.8) (layer F.Cu) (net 13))
 (segment (start 195.75 111.465) (end 195.41 111.125) (width 0.8) (layer F.Cu) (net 13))
 (segment (start 198.12 103.632) (end 198.12 106.85) (width 0.8) (layer F.Cu) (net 14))
 (segment (start 197.95 113.03) (end 197.95 111.465) (width 0.8) (layer F.Cu) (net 15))
 (segment (start 197.95 111.465) (end 198.29 111.125) (width 0.8) (layer F.Cu) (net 15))
 (segment (start 198.12 109.05) (end 198.12 110.955) (width 0.8) (layer F.Cu) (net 15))
 (segment (start 198.12 110.955) (end 198.29 111.125) (width 0.8) (layer F.Cu) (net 15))
 (segment (start 200.66 103.632) (end 200.66 106.85) (width 0.8) (layer F.Cu) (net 16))
 (segment (start 200.66 109.05) (end 201.91 109.05) (width 0.8) (layer F.Cu) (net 17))
 (segment (start 201.91 109.05) (end 203.2 107.76) (width 0.8) (layer F.Cu) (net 17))
 (segment (start 203.2 107.76) (end 203.2 106.51) (width 0.8) (layer F.Cu) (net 17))
 (segment (start 200.49 111.125) (end 200.49 109.22) (width 0.8) (layer F.Cu) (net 17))
 (segment (start 200.49 109.22) (end 200.66 109.05) (width 0.8) (layer F.Cu) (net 17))
 (segment (start 203.2 103.632) (end 203.2 106.51) (width 0.8) (layer F.Cu) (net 17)))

